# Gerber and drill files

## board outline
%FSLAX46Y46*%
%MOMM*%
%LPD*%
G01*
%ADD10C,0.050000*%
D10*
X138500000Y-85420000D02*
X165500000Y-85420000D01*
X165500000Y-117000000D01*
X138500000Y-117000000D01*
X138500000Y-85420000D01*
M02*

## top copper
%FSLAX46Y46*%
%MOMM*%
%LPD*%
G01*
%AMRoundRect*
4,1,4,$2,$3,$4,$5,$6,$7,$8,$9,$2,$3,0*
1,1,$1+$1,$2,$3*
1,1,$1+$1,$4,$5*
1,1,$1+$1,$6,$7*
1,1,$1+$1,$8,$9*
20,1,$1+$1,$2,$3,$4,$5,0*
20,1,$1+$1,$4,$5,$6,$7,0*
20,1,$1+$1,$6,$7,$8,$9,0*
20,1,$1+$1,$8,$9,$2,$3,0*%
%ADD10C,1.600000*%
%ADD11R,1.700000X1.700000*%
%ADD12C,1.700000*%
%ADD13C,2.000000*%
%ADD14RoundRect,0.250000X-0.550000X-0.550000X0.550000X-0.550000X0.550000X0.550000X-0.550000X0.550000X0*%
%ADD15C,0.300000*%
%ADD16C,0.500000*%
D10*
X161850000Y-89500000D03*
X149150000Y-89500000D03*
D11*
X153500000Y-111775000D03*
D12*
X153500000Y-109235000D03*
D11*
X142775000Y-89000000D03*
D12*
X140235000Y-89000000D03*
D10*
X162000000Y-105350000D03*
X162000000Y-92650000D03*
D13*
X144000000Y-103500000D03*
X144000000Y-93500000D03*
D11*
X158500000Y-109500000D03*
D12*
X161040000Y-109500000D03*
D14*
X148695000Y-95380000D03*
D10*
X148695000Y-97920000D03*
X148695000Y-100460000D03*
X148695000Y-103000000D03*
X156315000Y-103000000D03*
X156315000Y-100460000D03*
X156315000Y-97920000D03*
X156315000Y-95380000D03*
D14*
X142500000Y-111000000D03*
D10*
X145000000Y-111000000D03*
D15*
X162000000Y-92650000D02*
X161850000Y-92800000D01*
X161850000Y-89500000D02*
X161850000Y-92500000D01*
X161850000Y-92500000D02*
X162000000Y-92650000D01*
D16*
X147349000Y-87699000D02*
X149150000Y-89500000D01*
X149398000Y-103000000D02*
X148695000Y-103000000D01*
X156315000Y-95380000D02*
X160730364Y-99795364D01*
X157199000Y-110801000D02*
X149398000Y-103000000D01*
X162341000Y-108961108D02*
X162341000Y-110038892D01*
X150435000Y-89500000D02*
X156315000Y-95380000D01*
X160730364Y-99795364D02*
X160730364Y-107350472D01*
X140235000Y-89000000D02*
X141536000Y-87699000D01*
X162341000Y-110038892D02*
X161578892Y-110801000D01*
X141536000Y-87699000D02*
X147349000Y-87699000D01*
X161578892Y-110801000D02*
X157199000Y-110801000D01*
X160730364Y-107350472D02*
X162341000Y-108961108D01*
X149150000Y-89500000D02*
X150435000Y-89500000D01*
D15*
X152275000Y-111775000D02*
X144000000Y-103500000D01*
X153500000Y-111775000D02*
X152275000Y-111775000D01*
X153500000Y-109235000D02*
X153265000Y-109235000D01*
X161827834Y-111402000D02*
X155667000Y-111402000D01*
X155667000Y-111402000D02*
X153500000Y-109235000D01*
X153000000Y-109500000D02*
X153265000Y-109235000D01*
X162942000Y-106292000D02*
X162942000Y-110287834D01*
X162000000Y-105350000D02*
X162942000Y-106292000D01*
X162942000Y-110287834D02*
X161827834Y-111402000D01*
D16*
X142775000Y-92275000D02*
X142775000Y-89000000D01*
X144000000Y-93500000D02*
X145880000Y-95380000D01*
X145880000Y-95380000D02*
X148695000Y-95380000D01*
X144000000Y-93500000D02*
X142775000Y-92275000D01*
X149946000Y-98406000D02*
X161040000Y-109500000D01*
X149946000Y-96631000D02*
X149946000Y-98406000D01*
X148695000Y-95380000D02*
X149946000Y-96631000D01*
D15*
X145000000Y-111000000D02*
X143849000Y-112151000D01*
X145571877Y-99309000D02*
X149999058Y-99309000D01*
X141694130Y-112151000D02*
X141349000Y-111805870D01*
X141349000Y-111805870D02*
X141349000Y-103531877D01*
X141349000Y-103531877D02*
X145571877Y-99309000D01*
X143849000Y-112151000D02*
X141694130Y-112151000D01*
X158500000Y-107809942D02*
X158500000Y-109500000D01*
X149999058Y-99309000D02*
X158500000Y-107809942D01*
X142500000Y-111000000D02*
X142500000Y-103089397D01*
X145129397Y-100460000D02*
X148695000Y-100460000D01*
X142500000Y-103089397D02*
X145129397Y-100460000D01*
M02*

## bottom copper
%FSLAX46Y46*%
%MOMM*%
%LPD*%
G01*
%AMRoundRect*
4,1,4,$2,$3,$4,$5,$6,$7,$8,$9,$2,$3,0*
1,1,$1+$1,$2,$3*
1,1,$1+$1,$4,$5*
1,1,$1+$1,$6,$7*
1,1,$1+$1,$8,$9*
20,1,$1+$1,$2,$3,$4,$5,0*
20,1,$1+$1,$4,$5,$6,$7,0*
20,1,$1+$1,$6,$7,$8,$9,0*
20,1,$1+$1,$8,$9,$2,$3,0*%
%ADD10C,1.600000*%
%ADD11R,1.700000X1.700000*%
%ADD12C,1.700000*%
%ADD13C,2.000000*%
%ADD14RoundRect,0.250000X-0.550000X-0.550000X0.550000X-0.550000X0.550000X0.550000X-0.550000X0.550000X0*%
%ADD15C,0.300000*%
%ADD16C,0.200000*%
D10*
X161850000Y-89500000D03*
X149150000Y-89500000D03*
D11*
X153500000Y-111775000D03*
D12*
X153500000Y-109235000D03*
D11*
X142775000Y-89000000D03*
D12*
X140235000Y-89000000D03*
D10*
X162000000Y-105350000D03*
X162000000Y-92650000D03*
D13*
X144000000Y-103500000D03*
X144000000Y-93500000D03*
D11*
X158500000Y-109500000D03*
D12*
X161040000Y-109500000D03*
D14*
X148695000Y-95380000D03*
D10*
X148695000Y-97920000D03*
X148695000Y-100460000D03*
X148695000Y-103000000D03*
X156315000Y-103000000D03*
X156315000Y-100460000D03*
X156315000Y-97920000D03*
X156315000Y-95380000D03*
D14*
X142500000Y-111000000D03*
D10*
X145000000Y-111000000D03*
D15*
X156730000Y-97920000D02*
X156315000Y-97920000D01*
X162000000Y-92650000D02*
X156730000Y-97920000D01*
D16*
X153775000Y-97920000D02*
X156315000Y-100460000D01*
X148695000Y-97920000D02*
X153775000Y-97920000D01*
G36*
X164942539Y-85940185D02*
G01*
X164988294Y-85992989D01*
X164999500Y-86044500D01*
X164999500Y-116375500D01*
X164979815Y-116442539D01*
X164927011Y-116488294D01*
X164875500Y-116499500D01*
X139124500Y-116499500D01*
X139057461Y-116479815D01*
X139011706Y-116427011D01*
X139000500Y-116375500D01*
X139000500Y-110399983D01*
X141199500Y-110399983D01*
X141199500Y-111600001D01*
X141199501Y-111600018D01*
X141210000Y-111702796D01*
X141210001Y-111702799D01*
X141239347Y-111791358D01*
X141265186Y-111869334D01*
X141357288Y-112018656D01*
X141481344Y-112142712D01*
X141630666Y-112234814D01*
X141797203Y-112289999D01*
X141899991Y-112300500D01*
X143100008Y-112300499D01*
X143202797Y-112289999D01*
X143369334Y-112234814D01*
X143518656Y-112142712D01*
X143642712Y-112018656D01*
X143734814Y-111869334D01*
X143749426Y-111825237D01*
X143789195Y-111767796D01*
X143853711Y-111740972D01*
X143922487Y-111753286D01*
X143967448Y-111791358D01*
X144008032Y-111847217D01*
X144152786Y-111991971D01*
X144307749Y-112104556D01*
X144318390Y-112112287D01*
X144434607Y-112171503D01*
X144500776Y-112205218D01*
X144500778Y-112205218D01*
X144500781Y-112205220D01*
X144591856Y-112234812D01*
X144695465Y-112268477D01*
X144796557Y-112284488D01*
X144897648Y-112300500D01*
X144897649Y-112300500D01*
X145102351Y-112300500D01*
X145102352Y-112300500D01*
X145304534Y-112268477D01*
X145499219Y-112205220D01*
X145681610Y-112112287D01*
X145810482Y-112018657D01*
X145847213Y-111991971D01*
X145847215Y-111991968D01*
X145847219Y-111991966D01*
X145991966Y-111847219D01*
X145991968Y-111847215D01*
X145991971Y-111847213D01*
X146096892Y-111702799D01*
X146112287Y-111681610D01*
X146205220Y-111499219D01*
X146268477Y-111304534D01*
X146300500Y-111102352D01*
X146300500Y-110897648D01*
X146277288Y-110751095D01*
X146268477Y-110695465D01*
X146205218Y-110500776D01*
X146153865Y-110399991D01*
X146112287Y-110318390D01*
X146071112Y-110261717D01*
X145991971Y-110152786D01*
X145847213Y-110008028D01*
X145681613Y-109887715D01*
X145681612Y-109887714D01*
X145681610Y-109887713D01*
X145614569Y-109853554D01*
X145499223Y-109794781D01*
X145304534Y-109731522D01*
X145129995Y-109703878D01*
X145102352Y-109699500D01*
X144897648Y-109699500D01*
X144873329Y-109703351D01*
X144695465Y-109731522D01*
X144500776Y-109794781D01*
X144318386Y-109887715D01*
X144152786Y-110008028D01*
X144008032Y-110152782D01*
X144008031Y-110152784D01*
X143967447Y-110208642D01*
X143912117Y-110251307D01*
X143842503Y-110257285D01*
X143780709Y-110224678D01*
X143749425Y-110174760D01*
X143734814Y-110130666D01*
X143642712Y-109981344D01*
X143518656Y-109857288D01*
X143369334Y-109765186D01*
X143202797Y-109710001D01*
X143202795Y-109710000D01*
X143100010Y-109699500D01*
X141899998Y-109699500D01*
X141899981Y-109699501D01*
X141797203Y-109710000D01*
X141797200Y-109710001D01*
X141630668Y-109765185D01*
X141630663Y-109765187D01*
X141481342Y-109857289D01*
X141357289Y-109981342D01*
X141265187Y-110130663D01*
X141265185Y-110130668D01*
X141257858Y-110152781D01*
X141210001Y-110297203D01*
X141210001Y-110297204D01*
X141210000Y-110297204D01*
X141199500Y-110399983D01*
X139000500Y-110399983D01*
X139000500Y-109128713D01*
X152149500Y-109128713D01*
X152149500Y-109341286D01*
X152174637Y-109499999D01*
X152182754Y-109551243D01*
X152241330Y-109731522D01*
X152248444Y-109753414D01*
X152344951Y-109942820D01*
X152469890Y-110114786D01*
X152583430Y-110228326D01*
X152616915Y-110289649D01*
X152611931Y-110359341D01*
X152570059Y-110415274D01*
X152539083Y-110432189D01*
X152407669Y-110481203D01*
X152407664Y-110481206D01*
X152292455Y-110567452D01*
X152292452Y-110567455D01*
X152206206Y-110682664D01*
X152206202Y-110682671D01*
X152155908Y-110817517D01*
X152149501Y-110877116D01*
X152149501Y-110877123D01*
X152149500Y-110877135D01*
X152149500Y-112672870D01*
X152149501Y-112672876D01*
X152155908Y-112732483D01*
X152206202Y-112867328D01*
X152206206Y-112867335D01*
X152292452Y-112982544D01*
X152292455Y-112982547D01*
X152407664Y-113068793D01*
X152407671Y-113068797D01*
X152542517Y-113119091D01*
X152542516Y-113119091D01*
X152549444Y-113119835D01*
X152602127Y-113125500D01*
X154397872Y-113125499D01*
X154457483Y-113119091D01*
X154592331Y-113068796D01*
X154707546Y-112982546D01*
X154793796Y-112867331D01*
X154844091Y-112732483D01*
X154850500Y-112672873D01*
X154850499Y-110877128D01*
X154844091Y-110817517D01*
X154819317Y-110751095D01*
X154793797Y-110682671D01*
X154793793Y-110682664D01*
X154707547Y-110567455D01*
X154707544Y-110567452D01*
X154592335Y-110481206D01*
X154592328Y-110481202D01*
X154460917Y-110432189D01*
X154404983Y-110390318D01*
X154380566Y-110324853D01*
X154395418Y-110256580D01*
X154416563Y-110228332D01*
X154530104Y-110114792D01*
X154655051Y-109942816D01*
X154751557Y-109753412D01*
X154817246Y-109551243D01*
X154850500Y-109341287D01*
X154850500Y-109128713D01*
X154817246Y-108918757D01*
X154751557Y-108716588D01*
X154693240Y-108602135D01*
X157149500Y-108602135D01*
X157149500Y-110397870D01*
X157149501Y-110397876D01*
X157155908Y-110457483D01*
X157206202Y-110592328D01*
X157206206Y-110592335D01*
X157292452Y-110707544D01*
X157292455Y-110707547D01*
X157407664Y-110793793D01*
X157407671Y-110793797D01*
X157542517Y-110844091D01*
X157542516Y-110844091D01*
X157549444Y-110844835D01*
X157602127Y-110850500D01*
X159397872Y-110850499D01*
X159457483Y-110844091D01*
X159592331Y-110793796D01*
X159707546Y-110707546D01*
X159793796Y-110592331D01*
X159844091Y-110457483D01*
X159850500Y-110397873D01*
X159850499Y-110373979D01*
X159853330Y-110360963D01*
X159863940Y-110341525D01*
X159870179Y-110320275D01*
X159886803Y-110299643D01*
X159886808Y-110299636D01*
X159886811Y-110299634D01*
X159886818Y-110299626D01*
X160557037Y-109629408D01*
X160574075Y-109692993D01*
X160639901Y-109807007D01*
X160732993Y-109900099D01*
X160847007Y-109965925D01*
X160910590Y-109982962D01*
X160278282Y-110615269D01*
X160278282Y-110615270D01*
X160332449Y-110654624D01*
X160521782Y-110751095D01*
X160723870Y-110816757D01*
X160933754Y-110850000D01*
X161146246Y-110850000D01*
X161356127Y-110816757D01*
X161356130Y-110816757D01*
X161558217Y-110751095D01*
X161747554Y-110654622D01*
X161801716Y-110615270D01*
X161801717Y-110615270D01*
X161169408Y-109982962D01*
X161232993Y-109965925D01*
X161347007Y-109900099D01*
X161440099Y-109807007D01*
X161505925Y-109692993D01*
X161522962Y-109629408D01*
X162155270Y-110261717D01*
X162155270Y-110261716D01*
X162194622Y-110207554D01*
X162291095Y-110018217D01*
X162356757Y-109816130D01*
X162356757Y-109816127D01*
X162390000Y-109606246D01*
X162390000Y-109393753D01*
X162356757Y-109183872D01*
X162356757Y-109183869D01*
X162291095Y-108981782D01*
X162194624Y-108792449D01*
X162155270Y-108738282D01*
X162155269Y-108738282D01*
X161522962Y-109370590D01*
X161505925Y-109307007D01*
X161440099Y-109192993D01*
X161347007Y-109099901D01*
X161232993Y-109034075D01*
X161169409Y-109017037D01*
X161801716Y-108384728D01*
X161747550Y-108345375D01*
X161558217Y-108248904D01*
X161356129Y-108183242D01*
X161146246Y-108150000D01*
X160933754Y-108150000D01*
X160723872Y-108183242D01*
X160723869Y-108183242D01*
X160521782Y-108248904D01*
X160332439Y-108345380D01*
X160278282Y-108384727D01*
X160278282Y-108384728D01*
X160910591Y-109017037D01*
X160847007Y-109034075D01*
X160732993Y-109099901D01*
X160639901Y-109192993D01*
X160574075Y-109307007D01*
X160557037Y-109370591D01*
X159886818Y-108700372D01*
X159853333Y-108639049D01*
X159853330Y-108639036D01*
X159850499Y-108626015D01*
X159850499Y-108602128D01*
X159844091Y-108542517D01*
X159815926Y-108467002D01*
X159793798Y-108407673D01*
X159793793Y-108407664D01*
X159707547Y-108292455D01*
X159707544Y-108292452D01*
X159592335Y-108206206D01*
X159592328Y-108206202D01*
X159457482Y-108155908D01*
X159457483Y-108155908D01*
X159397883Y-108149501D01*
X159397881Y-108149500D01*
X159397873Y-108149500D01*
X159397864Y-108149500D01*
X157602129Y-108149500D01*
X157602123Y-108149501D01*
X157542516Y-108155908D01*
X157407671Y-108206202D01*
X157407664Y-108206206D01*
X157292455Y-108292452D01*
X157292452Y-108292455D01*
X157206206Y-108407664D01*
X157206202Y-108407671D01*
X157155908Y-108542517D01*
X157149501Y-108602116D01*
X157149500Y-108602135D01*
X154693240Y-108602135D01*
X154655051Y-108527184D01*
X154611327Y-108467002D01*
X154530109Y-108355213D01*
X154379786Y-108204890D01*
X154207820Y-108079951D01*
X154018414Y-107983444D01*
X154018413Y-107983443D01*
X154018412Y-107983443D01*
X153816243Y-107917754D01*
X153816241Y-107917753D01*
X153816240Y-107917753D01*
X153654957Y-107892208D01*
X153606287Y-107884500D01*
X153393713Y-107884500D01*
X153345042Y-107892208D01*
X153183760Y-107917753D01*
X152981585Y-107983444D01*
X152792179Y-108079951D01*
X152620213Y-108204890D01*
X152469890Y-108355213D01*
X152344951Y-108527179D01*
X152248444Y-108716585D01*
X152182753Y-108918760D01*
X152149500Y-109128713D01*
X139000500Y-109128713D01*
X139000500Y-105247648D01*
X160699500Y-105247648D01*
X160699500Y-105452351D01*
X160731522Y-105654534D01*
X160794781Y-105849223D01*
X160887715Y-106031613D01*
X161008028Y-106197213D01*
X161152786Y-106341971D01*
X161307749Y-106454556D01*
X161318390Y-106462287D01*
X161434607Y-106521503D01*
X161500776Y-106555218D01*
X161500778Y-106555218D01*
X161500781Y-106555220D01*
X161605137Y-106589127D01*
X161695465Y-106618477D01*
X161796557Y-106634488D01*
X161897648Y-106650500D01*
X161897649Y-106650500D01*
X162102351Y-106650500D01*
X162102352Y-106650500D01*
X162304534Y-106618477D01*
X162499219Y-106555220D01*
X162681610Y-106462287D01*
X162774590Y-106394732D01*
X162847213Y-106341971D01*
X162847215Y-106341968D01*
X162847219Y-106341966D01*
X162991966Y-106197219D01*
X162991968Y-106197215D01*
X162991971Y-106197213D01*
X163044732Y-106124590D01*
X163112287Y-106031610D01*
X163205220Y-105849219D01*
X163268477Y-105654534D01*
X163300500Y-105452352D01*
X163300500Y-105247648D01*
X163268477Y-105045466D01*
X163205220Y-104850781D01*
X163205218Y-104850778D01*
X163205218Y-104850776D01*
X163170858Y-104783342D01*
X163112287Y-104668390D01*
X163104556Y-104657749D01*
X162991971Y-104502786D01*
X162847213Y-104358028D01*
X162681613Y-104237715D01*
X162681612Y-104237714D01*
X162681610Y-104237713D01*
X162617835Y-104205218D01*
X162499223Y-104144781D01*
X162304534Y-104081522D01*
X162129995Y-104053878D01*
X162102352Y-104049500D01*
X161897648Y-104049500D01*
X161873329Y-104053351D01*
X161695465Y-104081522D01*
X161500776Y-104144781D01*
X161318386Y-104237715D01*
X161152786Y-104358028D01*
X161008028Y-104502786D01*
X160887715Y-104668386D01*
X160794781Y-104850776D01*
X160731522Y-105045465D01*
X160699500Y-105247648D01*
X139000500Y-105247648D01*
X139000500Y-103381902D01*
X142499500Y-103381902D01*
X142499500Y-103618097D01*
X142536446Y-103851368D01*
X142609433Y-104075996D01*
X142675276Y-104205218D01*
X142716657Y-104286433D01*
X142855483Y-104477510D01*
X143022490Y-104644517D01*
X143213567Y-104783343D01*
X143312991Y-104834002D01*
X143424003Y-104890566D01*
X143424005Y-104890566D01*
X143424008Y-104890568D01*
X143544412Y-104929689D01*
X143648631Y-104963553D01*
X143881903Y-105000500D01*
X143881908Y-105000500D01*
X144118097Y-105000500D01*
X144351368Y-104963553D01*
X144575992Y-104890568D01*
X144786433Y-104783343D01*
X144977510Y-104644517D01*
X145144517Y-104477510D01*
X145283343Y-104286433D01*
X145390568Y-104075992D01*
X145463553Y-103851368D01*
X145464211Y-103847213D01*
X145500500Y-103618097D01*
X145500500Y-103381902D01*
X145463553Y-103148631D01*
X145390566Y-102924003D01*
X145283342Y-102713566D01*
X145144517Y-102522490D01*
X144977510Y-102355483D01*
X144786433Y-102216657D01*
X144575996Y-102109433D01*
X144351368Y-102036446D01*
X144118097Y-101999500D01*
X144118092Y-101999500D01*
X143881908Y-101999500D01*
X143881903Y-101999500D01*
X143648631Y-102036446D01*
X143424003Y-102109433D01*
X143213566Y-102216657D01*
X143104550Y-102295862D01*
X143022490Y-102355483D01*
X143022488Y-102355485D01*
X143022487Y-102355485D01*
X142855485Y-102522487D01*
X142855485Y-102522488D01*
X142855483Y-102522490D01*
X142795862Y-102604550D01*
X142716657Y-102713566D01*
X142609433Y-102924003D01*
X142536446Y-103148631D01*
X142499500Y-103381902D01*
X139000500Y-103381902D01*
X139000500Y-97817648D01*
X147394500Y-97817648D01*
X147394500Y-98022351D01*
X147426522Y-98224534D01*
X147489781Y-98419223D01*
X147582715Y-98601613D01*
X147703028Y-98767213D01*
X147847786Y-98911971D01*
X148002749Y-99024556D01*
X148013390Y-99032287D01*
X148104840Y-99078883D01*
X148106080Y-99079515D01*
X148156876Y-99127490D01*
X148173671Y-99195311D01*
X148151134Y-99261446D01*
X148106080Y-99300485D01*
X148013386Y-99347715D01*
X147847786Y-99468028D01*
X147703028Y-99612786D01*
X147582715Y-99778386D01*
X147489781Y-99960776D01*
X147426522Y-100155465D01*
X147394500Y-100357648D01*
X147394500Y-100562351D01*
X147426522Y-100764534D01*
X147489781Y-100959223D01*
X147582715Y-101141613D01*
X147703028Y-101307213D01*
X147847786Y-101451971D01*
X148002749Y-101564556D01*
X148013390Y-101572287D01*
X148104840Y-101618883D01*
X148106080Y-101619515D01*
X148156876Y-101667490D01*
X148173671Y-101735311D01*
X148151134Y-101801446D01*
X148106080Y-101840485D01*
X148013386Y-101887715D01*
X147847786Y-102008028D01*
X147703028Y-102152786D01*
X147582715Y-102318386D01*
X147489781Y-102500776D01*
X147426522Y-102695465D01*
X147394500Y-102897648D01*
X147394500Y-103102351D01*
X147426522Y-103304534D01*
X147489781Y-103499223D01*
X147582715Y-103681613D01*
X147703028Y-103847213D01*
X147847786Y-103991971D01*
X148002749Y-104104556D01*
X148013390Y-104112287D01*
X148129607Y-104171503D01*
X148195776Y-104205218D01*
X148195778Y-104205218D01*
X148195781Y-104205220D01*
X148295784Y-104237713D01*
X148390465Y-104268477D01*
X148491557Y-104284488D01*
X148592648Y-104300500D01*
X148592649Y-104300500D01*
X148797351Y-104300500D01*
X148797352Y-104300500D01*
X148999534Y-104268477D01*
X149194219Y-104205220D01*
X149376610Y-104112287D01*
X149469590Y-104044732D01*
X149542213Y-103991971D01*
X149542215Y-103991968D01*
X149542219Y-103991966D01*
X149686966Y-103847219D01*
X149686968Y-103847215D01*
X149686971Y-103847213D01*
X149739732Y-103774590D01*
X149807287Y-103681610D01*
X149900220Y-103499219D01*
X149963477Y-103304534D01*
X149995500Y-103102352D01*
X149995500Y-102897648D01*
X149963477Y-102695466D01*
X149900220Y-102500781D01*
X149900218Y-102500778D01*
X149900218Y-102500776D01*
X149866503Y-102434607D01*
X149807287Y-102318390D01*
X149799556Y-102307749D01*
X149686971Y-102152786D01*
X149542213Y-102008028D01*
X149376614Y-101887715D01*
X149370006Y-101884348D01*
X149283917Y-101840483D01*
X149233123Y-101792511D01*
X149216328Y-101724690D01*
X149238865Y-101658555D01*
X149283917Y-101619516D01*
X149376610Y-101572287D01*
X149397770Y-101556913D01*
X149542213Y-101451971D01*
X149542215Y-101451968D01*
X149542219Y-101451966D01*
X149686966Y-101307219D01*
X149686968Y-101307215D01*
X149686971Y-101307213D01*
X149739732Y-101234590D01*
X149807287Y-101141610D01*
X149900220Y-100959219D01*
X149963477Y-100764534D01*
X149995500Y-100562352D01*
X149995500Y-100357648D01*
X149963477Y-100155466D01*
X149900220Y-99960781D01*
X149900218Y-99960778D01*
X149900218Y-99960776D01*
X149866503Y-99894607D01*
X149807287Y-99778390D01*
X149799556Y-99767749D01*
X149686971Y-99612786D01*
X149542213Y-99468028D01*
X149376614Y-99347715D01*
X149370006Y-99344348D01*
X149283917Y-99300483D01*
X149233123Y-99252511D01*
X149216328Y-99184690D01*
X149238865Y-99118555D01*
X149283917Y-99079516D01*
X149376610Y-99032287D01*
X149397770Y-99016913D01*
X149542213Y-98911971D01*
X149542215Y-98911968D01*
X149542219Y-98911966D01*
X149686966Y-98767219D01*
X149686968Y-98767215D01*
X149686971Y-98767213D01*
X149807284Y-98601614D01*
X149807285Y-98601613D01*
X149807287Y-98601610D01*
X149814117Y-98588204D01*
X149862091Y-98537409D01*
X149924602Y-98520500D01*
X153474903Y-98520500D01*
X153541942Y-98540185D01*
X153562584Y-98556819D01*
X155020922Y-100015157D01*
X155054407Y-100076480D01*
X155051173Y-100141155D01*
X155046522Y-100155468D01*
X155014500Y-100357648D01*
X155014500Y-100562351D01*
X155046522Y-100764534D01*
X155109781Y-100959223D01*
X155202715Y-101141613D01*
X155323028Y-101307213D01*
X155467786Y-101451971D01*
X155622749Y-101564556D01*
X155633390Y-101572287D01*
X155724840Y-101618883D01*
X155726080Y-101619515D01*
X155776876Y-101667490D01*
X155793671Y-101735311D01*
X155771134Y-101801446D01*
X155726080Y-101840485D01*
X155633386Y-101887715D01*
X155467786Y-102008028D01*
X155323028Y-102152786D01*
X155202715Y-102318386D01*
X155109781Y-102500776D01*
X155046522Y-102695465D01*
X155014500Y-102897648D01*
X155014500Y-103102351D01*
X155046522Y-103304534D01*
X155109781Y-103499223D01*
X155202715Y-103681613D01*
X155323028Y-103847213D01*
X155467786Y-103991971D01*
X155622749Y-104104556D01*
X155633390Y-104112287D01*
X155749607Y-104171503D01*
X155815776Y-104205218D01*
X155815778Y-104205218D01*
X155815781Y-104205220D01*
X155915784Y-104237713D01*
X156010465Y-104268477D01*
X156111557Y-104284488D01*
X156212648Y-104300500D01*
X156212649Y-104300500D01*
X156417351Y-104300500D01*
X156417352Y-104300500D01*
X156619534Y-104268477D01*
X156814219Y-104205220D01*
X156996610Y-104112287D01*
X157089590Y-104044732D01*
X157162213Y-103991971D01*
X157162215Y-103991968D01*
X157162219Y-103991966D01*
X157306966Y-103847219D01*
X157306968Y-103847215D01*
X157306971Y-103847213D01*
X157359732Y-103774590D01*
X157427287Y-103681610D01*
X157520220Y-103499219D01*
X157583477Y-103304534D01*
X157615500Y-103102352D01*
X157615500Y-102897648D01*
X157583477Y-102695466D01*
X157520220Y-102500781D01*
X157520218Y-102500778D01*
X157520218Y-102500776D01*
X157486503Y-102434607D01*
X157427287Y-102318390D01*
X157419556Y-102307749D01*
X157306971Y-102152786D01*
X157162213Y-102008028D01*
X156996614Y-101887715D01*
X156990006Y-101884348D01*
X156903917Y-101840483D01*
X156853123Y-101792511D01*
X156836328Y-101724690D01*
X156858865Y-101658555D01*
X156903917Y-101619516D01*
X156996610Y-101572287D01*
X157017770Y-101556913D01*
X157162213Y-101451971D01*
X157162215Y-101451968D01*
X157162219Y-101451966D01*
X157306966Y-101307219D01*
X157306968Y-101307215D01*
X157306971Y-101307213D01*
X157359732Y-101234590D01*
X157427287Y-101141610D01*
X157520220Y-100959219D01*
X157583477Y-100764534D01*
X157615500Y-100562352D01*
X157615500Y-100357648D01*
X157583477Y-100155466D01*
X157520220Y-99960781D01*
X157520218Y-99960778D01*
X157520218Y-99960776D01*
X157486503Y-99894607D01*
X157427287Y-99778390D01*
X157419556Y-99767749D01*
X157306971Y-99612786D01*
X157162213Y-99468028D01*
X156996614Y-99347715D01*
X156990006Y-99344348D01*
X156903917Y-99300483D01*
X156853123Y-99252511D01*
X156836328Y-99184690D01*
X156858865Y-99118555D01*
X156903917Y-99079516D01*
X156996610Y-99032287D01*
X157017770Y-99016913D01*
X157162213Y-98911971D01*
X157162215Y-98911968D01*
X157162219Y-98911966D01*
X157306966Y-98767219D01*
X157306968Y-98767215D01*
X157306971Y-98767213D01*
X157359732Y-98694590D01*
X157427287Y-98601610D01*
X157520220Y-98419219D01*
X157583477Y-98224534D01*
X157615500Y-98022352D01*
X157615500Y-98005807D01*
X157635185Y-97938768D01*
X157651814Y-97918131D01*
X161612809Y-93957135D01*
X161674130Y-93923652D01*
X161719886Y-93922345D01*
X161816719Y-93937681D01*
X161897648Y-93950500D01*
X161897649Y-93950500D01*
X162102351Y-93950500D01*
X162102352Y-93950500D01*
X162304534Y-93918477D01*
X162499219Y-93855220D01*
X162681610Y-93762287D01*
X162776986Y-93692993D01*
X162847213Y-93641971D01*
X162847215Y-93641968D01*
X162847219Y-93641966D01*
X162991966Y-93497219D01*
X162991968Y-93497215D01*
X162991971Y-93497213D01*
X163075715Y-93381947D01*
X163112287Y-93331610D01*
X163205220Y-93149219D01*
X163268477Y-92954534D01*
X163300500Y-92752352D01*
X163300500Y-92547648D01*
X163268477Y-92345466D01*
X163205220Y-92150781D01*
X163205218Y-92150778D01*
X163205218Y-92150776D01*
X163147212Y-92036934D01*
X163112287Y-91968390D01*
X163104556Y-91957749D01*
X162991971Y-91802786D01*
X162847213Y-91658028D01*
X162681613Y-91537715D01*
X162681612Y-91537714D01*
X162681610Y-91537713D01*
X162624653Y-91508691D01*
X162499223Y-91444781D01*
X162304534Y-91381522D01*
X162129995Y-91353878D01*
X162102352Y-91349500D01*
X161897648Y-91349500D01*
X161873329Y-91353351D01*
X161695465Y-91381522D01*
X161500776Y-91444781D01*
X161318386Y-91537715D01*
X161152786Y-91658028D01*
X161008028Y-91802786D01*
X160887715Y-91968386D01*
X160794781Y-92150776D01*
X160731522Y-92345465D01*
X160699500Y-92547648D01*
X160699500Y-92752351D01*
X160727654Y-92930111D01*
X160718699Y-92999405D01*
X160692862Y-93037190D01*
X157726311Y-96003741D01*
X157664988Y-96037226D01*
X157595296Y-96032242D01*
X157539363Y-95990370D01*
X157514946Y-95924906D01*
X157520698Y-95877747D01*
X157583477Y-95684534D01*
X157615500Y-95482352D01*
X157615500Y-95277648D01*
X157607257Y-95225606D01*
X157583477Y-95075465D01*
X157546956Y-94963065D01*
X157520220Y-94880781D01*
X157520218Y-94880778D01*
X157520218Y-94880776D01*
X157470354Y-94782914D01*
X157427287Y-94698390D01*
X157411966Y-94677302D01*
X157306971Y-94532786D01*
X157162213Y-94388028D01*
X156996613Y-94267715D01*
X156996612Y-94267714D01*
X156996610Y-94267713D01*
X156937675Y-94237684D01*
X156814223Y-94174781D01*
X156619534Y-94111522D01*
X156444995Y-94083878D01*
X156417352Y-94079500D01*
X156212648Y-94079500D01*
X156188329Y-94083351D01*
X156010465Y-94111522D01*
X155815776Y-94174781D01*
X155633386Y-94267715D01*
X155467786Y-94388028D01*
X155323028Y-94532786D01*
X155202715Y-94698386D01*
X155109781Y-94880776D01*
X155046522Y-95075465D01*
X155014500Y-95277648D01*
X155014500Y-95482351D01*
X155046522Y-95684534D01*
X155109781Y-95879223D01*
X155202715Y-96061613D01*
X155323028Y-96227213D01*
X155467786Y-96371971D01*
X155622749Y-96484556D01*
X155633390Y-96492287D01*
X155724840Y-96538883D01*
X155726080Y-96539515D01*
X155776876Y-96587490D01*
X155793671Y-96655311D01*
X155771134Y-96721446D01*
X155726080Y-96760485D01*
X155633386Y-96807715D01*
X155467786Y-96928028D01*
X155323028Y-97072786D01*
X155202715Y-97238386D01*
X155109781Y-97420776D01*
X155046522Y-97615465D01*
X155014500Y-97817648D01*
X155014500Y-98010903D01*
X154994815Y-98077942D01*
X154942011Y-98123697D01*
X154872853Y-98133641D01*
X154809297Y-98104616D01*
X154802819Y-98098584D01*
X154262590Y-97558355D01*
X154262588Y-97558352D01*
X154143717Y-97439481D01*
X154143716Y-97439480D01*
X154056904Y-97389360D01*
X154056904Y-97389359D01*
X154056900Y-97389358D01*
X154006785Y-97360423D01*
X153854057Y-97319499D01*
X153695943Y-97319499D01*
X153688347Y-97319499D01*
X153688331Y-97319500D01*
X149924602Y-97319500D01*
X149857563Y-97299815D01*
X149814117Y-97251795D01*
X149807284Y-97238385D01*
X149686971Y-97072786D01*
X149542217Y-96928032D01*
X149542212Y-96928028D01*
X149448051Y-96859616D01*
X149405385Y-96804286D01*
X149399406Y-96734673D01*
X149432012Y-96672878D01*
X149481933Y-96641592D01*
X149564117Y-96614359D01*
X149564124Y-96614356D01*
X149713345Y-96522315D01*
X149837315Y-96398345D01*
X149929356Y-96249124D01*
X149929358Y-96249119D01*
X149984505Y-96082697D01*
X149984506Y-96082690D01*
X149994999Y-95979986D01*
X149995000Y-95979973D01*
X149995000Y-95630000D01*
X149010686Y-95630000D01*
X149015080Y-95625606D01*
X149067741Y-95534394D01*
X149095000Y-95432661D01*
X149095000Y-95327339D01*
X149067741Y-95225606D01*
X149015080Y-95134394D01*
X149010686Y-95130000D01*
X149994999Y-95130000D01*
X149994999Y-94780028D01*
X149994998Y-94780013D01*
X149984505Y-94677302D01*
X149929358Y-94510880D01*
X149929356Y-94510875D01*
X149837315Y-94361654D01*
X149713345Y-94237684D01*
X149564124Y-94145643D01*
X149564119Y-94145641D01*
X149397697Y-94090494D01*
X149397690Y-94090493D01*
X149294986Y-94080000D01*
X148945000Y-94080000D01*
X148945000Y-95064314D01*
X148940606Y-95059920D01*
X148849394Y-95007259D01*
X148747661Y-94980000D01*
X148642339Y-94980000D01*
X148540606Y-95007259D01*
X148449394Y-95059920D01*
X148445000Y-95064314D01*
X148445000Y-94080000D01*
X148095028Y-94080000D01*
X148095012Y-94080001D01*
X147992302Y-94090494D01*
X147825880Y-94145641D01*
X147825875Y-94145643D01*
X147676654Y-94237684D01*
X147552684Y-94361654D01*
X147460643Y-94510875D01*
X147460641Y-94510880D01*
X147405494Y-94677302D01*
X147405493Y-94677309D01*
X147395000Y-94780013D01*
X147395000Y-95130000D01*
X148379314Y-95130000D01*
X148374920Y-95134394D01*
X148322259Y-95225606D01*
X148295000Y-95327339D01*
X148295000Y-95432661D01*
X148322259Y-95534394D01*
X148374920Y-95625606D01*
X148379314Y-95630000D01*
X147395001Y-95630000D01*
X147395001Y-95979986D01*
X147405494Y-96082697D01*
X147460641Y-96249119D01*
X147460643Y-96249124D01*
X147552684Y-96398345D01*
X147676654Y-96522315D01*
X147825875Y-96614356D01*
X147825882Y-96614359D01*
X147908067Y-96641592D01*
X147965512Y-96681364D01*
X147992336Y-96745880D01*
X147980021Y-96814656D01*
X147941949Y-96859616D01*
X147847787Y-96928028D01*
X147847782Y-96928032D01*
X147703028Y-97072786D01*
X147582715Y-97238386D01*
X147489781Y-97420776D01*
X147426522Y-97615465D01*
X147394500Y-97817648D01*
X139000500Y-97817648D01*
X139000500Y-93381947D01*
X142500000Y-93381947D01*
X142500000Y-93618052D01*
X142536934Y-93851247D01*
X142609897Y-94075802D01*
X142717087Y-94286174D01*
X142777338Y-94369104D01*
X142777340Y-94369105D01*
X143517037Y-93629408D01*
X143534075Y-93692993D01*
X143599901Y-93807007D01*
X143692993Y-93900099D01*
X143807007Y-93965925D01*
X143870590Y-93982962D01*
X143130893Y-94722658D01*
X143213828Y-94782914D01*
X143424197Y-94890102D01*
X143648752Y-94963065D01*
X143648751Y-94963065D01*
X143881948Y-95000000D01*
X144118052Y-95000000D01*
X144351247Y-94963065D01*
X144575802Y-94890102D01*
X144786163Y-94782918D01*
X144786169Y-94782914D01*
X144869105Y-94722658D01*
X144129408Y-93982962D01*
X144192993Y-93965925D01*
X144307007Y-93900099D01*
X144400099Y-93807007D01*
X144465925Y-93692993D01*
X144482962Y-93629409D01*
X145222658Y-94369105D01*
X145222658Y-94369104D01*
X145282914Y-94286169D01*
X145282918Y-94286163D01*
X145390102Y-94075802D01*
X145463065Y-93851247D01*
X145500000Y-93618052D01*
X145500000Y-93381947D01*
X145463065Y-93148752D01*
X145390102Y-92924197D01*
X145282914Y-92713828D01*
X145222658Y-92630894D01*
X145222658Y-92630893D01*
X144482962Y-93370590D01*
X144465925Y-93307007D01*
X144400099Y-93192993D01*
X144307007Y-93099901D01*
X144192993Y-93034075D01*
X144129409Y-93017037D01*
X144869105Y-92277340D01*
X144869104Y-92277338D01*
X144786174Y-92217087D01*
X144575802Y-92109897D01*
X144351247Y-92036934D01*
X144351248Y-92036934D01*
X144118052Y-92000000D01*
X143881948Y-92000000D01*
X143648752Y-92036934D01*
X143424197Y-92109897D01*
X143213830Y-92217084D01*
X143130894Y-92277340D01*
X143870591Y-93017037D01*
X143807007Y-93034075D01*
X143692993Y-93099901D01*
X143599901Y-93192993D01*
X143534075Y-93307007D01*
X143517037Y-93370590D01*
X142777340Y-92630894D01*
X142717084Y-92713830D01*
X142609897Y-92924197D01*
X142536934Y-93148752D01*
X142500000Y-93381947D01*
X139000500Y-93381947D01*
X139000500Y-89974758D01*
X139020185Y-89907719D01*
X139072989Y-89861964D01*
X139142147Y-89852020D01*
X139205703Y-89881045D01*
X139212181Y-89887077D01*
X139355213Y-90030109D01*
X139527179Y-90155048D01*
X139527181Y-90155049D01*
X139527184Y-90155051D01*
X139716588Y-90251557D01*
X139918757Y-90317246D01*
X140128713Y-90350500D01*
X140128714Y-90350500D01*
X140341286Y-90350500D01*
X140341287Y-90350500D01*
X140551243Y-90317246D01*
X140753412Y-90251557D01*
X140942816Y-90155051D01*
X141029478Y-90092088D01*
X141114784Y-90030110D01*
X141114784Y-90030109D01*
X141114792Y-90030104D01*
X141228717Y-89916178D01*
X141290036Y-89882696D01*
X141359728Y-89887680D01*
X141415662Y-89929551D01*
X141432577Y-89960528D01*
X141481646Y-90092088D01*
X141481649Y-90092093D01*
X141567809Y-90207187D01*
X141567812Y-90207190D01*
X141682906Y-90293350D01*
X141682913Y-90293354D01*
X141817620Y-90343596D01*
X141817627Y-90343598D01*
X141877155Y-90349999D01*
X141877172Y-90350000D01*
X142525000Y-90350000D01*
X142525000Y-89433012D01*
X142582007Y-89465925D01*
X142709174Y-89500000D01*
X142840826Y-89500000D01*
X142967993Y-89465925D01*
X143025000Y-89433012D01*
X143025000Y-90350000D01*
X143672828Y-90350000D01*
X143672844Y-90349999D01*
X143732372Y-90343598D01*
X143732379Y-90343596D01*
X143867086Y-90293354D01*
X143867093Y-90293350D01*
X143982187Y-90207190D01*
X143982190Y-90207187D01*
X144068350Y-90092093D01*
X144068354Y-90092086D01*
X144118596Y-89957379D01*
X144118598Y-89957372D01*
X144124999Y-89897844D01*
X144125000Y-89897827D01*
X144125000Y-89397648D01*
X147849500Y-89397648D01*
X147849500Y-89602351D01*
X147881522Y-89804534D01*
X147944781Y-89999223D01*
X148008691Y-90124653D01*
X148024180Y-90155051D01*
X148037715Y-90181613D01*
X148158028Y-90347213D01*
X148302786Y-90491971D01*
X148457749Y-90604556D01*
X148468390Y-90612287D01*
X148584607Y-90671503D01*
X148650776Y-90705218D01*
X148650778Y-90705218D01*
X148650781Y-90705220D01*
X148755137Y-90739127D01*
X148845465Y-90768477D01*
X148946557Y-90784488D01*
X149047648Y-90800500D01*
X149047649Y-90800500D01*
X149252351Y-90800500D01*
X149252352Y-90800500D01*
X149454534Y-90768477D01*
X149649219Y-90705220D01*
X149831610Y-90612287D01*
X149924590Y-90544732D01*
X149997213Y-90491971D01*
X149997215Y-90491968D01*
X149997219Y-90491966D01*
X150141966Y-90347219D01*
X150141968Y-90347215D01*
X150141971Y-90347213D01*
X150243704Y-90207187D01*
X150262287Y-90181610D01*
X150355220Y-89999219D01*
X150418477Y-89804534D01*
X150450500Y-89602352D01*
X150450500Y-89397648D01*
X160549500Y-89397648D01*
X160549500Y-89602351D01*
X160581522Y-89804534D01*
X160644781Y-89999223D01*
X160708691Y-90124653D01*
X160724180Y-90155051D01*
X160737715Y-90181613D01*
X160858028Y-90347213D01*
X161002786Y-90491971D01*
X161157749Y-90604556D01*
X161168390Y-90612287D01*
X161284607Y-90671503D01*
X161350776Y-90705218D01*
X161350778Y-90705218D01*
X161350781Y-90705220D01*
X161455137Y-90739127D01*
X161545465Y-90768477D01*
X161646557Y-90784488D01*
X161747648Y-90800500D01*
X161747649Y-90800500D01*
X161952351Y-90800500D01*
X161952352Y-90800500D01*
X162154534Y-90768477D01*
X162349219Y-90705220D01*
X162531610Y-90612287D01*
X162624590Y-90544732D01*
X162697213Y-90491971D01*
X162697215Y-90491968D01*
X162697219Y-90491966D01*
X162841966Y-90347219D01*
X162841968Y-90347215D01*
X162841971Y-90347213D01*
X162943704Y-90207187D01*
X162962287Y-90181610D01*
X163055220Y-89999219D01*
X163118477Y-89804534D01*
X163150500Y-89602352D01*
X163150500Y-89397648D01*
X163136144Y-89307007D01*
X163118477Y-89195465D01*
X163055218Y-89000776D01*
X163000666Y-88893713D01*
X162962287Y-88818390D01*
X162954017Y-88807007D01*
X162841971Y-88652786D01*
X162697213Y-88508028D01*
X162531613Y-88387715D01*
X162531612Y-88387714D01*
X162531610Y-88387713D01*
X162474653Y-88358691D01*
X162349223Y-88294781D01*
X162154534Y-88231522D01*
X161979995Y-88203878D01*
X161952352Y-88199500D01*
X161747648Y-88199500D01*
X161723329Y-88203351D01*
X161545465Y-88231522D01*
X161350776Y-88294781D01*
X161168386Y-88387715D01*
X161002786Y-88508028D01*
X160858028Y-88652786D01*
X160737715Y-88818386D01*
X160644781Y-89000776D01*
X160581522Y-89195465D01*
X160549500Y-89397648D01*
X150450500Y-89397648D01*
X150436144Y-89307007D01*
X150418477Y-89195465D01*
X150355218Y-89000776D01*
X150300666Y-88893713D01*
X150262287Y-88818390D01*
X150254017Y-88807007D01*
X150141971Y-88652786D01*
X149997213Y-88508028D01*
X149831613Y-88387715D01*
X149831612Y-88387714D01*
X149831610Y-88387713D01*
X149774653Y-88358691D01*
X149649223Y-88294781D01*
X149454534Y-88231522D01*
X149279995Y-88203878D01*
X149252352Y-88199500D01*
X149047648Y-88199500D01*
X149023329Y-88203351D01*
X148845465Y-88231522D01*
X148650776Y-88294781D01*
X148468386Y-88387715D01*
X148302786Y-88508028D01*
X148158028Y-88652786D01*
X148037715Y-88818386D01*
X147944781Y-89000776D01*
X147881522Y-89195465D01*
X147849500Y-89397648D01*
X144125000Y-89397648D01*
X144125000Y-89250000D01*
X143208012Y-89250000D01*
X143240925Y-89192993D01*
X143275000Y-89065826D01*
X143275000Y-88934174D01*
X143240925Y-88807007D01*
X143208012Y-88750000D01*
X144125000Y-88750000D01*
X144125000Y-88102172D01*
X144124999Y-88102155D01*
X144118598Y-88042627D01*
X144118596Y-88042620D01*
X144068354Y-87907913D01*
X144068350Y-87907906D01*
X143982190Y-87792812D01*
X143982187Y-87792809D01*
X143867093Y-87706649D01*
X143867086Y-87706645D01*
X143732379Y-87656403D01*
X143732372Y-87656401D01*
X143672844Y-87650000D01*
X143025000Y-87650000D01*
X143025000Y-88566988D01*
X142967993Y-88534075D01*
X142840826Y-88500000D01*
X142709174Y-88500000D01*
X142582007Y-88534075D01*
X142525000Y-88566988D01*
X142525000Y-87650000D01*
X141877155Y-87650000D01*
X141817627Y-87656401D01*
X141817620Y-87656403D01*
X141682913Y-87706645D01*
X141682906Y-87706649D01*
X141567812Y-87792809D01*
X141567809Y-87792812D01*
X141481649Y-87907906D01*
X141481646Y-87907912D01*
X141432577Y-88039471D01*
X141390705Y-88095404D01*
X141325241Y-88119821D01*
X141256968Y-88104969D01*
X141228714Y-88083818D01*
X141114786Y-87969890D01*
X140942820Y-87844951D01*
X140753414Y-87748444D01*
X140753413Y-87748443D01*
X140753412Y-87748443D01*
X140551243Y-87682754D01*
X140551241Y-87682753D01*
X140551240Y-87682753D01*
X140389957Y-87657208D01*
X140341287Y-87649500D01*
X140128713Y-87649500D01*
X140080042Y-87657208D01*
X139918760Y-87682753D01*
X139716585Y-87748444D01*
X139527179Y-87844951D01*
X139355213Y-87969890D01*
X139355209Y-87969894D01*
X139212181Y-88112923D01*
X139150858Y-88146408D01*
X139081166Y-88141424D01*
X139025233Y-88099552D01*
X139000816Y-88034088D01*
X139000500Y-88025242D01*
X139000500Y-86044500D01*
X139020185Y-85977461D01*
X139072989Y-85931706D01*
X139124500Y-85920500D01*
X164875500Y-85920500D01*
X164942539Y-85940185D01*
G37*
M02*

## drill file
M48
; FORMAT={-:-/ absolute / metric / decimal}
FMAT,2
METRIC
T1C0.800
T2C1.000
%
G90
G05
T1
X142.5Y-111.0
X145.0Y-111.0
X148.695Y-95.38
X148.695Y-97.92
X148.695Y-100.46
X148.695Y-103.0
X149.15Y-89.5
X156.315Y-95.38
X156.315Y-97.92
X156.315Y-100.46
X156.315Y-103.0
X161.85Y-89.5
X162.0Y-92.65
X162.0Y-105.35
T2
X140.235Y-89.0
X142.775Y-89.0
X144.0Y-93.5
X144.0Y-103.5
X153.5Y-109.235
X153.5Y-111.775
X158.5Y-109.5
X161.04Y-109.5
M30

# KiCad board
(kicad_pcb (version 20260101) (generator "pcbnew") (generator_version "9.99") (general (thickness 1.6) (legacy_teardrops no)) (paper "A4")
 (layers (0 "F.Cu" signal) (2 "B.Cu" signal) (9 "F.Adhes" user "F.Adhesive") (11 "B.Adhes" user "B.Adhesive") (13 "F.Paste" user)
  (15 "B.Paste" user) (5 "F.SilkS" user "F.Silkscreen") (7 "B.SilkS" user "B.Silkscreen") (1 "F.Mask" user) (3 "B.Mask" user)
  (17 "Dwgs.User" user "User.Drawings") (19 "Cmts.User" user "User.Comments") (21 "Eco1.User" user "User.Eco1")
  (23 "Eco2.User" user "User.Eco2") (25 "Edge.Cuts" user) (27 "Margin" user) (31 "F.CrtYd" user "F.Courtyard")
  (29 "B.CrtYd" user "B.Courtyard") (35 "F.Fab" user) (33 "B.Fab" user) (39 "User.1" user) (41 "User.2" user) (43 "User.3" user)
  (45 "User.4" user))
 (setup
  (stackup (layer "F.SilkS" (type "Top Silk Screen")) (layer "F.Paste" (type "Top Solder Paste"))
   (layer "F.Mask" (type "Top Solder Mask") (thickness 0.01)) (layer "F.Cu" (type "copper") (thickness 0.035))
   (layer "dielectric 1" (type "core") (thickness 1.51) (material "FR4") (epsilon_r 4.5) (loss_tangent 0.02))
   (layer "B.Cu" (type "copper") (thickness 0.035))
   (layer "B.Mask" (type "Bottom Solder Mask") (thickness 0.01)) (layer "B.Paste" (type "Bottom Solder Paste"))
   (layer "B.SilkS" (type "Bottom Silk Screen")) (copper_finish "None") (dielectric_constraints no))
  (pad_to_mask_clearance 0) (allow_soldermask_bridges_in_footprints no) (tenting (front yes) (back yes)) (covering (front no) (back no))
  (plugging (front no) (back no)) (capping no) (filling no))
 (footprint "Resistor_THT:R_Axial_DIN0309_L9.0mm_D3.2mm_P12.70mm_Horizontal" (layer "F.Cu") (at 161.85 89.5 180)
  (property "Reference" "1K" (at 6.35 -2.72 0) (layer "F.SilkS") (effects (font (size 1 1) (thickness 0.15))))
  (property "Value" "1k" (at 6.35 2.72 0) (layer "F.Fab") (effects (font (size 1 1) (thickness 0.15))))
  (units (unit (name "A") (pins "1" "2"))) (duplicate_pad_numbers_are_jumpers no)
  (pad "1" thru_hole circle (at 0 0 180) (size 1.6 1.6) (drill 0.8) (layers "*.Cu" "*.Mask") (remove_unused_layers no) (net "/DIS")
   (tenting (front none) (back none)))
  (pad "2" thru_hole circle (at 12.7 0 180) (size 1.6 1.6) (drill 0.8) (layers "*.Cu" "*.Mask") (remove_unused_layers no) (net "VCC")
   (tenting (front none) (back none))))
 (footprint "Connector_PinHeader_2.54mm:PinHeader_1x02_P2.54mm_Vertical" (layer "F.Cu") (at 153.5 111.775 180)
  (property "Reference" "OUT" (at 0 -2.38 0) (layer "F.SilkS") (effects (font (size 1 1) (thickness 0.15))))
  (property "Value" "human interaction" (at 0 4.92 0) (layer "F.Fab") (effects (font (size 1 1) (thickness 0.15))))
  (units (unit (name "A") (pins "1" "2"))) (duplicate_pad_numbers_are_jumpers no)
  (pad "1" thru_hole rect (at 0 0 180) (size 1.7 1.7) (drill 1) (layers "*.Cu" "*.Mask") (remove_unused_layers no) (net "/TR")
   (tenting (front none) (back none)))
  (pad "2" thru_hole circle (at 0 2.54 180) (size 1.7 1.7) (drill 1) (layers "*.Cu" "*.Mask") (remove_unused_layers no)
   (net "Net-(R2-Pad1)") (tenting (front none) (back none))))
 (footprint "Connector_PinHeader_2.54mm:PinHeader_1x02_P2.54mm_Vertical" (layer "F.Cu") (at 142.775 89 -90)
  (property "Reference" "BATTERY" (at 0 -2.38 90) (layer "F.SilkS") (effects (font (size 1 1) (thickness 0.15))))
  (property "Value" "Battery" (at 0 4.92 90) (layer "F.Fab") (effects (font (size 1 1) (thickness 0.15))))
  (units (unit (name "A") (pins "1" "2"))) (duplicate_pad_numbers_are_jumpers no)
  (pad "1" thru_hole rect (at 0 0 270) (size 1.7 1.7) (drill 1) (layers "*.Cu" "*.Mask") (remove_unused_layers no) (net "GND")
   (tenting (front none) (back none)))
  (pad "2" thru_hole circle (at 0 2.54 270) (size 1.7 1.7) (drill 1) (layers "*.Cu" "*.Mask") (remove_unused_layers no) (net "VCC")
   (tenting (front none) (back none))))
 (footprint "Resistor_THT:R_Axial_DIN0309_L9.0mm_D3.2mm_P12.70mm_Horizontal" (layer "F.Cu") (at 162 105.35 90)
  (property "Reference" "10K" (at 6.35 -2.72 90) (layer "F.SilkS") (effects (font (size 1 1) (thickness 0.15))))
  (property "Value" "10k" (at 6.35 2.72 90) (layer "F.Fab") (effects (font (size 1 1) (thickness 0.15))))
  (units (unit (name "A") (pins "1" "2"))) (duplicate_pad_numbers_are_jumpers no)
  (pad "1" thru_hole circle (at 0 0 90) (size 1.6 1.6) (drill 0.8) (layers "*.Cu" "*.Mask") (remove_unused_layers no) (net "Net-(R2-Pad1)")
   (tenting (front none) (back none)))
  (pad "2" thru_hole circle (at 12.7 0 90) (size 1.6 1.6) (drill 0.8) (layers "*.Cu" "*.Mask") (remove_unused_layers no) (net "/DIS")
   (tenting (front none) (back none))))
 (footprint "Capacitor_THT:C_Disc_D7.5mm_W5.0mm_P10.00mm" (layer "F.Cu") (at 144 103.5 90)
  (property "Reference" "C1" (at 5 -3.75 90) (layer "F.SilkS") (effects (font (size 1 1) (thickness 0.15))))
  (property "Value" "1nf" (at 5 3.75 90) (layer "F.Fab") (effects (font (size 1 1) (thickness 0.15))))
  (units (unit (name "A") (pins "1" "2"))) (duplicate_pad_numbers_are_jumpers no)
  (pad "1" thru_hole circle (at 0 0 90) (size 2 2) (drill 1) (layers "*.Cu" "*.Mask") (remove_unused_layers no) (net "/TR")
   (tenting (front none) (back none)))
  (pad "2" thru_hole circle (at 10 0 90) (size 2 2) (drill 1) (layers "*.Cu" "*.Mask") (remove_unused_layers no) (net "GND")
   (tenting (front none) (back none))))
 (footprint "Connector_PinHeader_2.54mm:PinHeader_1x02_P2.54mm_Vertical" (layer "F.Cu") (at 158.5 109.5 90)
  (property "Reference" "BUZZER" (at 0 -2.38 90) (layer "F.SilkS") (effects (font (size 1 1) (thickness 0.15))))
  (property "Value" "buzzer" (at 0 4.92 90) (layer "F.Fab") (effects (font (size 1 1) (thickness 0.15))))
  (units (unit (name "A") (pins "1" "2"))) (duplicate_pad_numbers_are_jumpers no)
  (pad "1" thru_hole rect (at 0 0 90) (size 1.7 1.7) (drill 1) (layers "*.Cu" "*.Mask") (remove_unused_layers no) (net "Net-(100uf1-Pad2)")
   (tenting (front none) (back none)))
  (pad "2" thru_hole circle (at 0 2.54 90) (size 1.7 1.7) (drill 1) (layers "*.Cu" "*.Mask") (remove_unused_layers no) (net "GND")
   (tenting (front none) (back none))))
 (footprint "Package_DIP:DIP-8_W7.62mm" (layer "F.Cu") (at 148.695 95.38)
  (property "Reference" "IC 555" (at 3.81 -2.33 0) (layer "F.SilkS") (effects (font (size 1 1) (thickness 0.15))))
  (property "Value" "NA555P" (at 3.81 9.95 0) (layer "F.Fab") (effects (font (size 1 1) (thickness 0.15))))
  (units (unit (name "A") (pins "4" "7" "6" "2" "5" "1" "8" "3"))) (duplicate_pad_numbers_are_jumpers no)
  (pad "1" thru_hole roundrect (at 0 0) (size 1.6 1.6) (drill 0.8) (layers "*.Cu" "*.Mask") (remove_unused_layers no)
   (roundrect_rratio 0.15625) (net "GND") (tenting (front none) (back none)))
  (pad "2" thru_hole circle (at 0 2.54) (size 1.6 1.6) (drill 0.8) (layers "*.Cu" "*.Mask") (remove_unused_layers no) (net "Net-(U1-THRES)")
   (tenting (front none) (back none)))
  (pad "3" thru_hole circle (at 0 5.08) (size 1.6 1.6) (drill 0.8) (layers "*.Cu" "*.Mask") (remove_unused_layers no) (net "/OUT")
   (tenting (front none) (back none)))
  (pad "4" thru_hole circle (at 0 7.62) (size 1.6 1.6) (drill 0.8) (layers "*.Cu" "*.Mask") (remove_unused_layers no) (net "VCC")
   (tenting (front none) (back none)))
  (pad "5" thru_hole circle (at 7.62 7.62) (size 1.6 1.6) (drill 0.8) (layers "*.Cu" "*.Mask") (remove_unused_layers no)
   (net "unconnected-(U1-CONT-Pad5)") (tenting (front none) (back none)))
  (pad "6" thru_hole circle (at 7.62 5.08) (size 1.6 1.6) (drill 0.8) (layers "*.Cu" "*.Mask") (remove_unused_layers no)
   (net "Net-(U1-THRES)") (tenting (front none) (back none)))
  (pad "7" thru_hole circle (at 7.62 2.54) (size 1.6 1.6) (drill 0.8) (layers "*.Cu" "*.Mask") (remove_unused_layers no) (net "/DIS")
   (tenting (front none) (back none)))
  (pad "8" thru_hole circle (at 7.62 0) (size 1.6 1.6) (drill 0.8) (layers "*.Cu" "*.Mask") (remove_unused_layers no) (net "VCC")
   (tenting (front none) (back none))))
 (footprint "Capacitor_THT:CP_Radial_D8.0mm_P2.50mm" (layer "F.Cu") (at 142.5 111)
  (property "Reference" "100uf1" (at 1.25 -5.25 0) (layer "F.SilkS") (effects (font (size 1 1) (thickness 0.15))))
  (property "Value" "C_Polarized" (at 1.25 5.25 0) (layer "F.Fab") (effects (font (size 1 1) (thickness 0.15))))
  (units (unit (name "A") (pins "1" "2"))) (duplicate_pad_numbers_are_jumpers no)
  (pad "1" thru_hole roundrect (at 0 0) (size 1.6 1.6) (drill 0.8) (layers "*.Cu" "*.Mask") (remove_unused_layers no)
   (roundrect_rratio 0.15625) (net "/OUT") (tenting (front none) (back none)))
  (pad "2" thru_hole circle (at 2.5 0) (size 1.6 1.6) (drill 0.8) (layers "*.Cu" "*.Mask") (remove_unused_layers no)
   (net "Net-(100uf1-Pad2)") (tenting (front none) (back none))))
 (gr_rect (start 138.5 85.42) (end 165.5 117) (stroke (width 0.05) (type solid)) (fill no) (layer "Edge.Cuts"))
 (segment (start 162 92.65) (end 161.85 92.8) (width 0.3) (layer "F.Cu") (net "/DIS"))
 (segment (start 161.85 89.5) (end 161.85 92.5) (width 0.3) (layer "F.Cu") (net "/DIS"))
 (segment (start 161.85 92.5) (end 162 92.65) (width 0.3) (layer "F.Cu") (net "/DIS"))
 (segment (start 156.73 97.92) (end 156.315 97.92) (width 0.3) (layer "B.Cu") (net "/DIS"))
 (segment (start 162 92.65) (end 156.73 97.92) (width 0.3) (layer "B.Cu") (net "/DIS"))
 (segment (start 147.349 87.699) (end 149.15 89.5) (width 0.5) (layer "F.Cu") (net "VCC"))
 (segment (start 149.398 103) (end 148.695 103) (width 0.5) (layer "F.Cu") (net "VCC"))
 (segment (start 156.315 95.38) (end 160.730364 99.795364) (width 0.5) (layer "F.Cu") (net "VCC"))
 (segment (start 157.199 110.801) (end 149.398 103) (width 0.5) (layer "F.Cu") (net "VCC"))
 (segment (start 162.341 108.961108) (end 162.341 110.038892) (width 0.5) (layer "F.Cu") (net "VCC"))
 (segment (start 150.435 89.5) (end 156.315 95.38) (width 0.5) (layer "F.Cu") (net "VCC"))
 (segment (start 160.730364 99.795364) (end 160.730364 107.350472) (width 0.5) (layer "F.Cu") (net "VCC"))
 (segment (start 140.235 89) (end 141.536 87.699) (width 0.5) (layer "F.Cu") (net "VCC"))
 (segment (start 162.341 110.038892) (end 161.578892 110.801) (width 0.5) (layer "F.Cu") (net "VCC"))
 (segment (start 141.536 87.699) (end 147.349 87.699) (width 0.5) (layer "F.Cu") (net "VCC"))
 (segment (start 161.578892 110.801) (end 157.199 110.801) (width 0.5) (layer "F.Cu") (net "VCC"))
 (segment (start 160.730364 107.350472) (end 162.341 108.961108) (width 0.5) (layer "F.Cu") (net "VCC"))
 (segment (start 149.15 89.5) (end 150.435 89.5) (width 0.5) (layer "F.Cu") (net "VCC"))
 (segment (start 152.275 111.775) (end 144 103.5) (width 0.3) (layer "F.Cu") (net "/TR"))
 (segment (start 153.5 111.775) (end 152.275 111.775) (width 0.3) (layer "F.Cu") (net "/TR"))
 (segment (start 153.5 109.235) (end 153.265 109.235) (width 0.3) (layer "F.Cu") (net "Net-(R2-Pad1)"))
 (segment (start 161.827834 111.402) (end 155.667 111.402) (width 0.3) (layer "F.Cu") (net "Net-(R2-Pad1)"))
 (segment (start 155.667 111.402) (end 153.5 109.235) (width 0.3) (layer "F.Cu") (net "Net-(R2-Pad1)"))
 (segment (start 153 109.5) (end 153.265 109.235) (width 0.3) (layer "F.Cu") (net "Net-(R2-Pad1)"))
 (segment (start 162.942 106.292) (end 162.942 110.287834) (width 0.3) (layer "F.Cu") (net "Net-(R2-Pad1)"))
 (segment (start 162 105.35) (end 162.942 106.292) (width 0.3) (layer "F.Cu") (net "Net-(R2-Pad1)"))
 (segment (start 162.942 110.287834) (end 161.827834 111.402) (width 0.3) (layer "F.Cu") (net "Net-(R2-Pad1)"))
 (segment (start 142.775 92.275) (end 142.775 89) (width 0.5) (layer "F.Cu") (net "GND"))
 (segment (start 144 93.5) (end 145.88 95.38) (width 0.5) (layer "F.Cu") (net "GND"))
 (segment (start 145.88 95.38) (end 148.695 95.38) (width 0.5) (layer "F.Cu") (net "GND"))
 (segment (start 144 93.5) (end 142.775 92.275) (width 0.5) (layer "F.Cu") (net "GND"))
 (segment (start 149.946 98.406) (end 161.04 109.5) (width 0.5) (layer "F.Cu") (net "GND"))
 (segment (start 149.946 96.631) (end 149.946 98.406) (width 0.5) (layer "F.Cu") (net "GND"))
 (segment (start 148.695 95.38) (end 149.946 96.631) (width 0.5) (layer "F.Cu") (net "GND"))
 (segment (start 145 111) (end 143.849 112.151) (width 0.3) (layer "F.Cu") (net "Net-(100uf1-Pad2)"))
 (segment (start 145.571877 99.309) (end 149.999058 99.309) (width 0.3) (layer "F.Cu") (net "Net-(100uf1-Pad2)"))
 (segment (start 141.69413 112.151) (end 141.349 111.80587) (width 0.3) (layer "F.Cu") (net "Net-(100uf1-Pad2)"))
 (segment (start 141.349 111.80587) (end 141.349 103.531877) (width 0.3) (layer "F.Cu") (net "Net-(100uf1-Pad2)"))
 (segment (start 141.349 103.531877) (end 145.571877 99.309) (width 0.3) (layer "F.Cu") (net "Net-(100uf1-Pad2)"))
 (segment (start 143.849 112.151) (end 141.69413 112.151) (width 0.3) (layer "F.Cu") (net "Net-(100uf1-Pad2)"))
 (segment (start 158.5 107.809942) (end 158.5 109.5) (width 0.3) (layer "F.Cu") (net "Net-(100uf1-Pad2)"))
 (segment (start 149.999058 99.309) (end 158.5 107.809942) (width 0.3) (layer "F.Cu") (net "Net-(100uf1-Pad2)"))
 (segment (start 153.775 97.92) (end 156.315 100.46) (width 0.2) (layer "B.Cu") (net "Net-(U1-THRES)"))
 (segment (start 148.695 97.92) (end 153.775 97.92) (width 0.2) (layer "B.Cu") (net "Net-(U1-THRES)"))
 (segment (start 142.5 111) (end 142.5 103.089397) (width 0.3) (layer "F.Cu") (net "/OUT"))
 (segment (start 145.129397 100.46) (end 148.695 100.46) (width 0.3) (layer "F.Cu") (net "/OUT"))
 (segment (start 142.5 103.089397) (end 145.129397 100.46) (width 0.3) (layer "F.Cu") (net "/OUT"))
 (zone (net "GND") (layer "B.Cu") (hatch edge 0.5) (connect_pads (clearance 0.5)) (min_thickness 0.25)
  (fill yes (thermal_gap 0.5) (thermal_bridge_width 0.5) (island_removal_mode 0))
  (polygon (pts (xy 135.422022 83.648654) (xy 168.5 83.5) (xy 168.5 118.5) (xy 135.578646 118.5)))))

